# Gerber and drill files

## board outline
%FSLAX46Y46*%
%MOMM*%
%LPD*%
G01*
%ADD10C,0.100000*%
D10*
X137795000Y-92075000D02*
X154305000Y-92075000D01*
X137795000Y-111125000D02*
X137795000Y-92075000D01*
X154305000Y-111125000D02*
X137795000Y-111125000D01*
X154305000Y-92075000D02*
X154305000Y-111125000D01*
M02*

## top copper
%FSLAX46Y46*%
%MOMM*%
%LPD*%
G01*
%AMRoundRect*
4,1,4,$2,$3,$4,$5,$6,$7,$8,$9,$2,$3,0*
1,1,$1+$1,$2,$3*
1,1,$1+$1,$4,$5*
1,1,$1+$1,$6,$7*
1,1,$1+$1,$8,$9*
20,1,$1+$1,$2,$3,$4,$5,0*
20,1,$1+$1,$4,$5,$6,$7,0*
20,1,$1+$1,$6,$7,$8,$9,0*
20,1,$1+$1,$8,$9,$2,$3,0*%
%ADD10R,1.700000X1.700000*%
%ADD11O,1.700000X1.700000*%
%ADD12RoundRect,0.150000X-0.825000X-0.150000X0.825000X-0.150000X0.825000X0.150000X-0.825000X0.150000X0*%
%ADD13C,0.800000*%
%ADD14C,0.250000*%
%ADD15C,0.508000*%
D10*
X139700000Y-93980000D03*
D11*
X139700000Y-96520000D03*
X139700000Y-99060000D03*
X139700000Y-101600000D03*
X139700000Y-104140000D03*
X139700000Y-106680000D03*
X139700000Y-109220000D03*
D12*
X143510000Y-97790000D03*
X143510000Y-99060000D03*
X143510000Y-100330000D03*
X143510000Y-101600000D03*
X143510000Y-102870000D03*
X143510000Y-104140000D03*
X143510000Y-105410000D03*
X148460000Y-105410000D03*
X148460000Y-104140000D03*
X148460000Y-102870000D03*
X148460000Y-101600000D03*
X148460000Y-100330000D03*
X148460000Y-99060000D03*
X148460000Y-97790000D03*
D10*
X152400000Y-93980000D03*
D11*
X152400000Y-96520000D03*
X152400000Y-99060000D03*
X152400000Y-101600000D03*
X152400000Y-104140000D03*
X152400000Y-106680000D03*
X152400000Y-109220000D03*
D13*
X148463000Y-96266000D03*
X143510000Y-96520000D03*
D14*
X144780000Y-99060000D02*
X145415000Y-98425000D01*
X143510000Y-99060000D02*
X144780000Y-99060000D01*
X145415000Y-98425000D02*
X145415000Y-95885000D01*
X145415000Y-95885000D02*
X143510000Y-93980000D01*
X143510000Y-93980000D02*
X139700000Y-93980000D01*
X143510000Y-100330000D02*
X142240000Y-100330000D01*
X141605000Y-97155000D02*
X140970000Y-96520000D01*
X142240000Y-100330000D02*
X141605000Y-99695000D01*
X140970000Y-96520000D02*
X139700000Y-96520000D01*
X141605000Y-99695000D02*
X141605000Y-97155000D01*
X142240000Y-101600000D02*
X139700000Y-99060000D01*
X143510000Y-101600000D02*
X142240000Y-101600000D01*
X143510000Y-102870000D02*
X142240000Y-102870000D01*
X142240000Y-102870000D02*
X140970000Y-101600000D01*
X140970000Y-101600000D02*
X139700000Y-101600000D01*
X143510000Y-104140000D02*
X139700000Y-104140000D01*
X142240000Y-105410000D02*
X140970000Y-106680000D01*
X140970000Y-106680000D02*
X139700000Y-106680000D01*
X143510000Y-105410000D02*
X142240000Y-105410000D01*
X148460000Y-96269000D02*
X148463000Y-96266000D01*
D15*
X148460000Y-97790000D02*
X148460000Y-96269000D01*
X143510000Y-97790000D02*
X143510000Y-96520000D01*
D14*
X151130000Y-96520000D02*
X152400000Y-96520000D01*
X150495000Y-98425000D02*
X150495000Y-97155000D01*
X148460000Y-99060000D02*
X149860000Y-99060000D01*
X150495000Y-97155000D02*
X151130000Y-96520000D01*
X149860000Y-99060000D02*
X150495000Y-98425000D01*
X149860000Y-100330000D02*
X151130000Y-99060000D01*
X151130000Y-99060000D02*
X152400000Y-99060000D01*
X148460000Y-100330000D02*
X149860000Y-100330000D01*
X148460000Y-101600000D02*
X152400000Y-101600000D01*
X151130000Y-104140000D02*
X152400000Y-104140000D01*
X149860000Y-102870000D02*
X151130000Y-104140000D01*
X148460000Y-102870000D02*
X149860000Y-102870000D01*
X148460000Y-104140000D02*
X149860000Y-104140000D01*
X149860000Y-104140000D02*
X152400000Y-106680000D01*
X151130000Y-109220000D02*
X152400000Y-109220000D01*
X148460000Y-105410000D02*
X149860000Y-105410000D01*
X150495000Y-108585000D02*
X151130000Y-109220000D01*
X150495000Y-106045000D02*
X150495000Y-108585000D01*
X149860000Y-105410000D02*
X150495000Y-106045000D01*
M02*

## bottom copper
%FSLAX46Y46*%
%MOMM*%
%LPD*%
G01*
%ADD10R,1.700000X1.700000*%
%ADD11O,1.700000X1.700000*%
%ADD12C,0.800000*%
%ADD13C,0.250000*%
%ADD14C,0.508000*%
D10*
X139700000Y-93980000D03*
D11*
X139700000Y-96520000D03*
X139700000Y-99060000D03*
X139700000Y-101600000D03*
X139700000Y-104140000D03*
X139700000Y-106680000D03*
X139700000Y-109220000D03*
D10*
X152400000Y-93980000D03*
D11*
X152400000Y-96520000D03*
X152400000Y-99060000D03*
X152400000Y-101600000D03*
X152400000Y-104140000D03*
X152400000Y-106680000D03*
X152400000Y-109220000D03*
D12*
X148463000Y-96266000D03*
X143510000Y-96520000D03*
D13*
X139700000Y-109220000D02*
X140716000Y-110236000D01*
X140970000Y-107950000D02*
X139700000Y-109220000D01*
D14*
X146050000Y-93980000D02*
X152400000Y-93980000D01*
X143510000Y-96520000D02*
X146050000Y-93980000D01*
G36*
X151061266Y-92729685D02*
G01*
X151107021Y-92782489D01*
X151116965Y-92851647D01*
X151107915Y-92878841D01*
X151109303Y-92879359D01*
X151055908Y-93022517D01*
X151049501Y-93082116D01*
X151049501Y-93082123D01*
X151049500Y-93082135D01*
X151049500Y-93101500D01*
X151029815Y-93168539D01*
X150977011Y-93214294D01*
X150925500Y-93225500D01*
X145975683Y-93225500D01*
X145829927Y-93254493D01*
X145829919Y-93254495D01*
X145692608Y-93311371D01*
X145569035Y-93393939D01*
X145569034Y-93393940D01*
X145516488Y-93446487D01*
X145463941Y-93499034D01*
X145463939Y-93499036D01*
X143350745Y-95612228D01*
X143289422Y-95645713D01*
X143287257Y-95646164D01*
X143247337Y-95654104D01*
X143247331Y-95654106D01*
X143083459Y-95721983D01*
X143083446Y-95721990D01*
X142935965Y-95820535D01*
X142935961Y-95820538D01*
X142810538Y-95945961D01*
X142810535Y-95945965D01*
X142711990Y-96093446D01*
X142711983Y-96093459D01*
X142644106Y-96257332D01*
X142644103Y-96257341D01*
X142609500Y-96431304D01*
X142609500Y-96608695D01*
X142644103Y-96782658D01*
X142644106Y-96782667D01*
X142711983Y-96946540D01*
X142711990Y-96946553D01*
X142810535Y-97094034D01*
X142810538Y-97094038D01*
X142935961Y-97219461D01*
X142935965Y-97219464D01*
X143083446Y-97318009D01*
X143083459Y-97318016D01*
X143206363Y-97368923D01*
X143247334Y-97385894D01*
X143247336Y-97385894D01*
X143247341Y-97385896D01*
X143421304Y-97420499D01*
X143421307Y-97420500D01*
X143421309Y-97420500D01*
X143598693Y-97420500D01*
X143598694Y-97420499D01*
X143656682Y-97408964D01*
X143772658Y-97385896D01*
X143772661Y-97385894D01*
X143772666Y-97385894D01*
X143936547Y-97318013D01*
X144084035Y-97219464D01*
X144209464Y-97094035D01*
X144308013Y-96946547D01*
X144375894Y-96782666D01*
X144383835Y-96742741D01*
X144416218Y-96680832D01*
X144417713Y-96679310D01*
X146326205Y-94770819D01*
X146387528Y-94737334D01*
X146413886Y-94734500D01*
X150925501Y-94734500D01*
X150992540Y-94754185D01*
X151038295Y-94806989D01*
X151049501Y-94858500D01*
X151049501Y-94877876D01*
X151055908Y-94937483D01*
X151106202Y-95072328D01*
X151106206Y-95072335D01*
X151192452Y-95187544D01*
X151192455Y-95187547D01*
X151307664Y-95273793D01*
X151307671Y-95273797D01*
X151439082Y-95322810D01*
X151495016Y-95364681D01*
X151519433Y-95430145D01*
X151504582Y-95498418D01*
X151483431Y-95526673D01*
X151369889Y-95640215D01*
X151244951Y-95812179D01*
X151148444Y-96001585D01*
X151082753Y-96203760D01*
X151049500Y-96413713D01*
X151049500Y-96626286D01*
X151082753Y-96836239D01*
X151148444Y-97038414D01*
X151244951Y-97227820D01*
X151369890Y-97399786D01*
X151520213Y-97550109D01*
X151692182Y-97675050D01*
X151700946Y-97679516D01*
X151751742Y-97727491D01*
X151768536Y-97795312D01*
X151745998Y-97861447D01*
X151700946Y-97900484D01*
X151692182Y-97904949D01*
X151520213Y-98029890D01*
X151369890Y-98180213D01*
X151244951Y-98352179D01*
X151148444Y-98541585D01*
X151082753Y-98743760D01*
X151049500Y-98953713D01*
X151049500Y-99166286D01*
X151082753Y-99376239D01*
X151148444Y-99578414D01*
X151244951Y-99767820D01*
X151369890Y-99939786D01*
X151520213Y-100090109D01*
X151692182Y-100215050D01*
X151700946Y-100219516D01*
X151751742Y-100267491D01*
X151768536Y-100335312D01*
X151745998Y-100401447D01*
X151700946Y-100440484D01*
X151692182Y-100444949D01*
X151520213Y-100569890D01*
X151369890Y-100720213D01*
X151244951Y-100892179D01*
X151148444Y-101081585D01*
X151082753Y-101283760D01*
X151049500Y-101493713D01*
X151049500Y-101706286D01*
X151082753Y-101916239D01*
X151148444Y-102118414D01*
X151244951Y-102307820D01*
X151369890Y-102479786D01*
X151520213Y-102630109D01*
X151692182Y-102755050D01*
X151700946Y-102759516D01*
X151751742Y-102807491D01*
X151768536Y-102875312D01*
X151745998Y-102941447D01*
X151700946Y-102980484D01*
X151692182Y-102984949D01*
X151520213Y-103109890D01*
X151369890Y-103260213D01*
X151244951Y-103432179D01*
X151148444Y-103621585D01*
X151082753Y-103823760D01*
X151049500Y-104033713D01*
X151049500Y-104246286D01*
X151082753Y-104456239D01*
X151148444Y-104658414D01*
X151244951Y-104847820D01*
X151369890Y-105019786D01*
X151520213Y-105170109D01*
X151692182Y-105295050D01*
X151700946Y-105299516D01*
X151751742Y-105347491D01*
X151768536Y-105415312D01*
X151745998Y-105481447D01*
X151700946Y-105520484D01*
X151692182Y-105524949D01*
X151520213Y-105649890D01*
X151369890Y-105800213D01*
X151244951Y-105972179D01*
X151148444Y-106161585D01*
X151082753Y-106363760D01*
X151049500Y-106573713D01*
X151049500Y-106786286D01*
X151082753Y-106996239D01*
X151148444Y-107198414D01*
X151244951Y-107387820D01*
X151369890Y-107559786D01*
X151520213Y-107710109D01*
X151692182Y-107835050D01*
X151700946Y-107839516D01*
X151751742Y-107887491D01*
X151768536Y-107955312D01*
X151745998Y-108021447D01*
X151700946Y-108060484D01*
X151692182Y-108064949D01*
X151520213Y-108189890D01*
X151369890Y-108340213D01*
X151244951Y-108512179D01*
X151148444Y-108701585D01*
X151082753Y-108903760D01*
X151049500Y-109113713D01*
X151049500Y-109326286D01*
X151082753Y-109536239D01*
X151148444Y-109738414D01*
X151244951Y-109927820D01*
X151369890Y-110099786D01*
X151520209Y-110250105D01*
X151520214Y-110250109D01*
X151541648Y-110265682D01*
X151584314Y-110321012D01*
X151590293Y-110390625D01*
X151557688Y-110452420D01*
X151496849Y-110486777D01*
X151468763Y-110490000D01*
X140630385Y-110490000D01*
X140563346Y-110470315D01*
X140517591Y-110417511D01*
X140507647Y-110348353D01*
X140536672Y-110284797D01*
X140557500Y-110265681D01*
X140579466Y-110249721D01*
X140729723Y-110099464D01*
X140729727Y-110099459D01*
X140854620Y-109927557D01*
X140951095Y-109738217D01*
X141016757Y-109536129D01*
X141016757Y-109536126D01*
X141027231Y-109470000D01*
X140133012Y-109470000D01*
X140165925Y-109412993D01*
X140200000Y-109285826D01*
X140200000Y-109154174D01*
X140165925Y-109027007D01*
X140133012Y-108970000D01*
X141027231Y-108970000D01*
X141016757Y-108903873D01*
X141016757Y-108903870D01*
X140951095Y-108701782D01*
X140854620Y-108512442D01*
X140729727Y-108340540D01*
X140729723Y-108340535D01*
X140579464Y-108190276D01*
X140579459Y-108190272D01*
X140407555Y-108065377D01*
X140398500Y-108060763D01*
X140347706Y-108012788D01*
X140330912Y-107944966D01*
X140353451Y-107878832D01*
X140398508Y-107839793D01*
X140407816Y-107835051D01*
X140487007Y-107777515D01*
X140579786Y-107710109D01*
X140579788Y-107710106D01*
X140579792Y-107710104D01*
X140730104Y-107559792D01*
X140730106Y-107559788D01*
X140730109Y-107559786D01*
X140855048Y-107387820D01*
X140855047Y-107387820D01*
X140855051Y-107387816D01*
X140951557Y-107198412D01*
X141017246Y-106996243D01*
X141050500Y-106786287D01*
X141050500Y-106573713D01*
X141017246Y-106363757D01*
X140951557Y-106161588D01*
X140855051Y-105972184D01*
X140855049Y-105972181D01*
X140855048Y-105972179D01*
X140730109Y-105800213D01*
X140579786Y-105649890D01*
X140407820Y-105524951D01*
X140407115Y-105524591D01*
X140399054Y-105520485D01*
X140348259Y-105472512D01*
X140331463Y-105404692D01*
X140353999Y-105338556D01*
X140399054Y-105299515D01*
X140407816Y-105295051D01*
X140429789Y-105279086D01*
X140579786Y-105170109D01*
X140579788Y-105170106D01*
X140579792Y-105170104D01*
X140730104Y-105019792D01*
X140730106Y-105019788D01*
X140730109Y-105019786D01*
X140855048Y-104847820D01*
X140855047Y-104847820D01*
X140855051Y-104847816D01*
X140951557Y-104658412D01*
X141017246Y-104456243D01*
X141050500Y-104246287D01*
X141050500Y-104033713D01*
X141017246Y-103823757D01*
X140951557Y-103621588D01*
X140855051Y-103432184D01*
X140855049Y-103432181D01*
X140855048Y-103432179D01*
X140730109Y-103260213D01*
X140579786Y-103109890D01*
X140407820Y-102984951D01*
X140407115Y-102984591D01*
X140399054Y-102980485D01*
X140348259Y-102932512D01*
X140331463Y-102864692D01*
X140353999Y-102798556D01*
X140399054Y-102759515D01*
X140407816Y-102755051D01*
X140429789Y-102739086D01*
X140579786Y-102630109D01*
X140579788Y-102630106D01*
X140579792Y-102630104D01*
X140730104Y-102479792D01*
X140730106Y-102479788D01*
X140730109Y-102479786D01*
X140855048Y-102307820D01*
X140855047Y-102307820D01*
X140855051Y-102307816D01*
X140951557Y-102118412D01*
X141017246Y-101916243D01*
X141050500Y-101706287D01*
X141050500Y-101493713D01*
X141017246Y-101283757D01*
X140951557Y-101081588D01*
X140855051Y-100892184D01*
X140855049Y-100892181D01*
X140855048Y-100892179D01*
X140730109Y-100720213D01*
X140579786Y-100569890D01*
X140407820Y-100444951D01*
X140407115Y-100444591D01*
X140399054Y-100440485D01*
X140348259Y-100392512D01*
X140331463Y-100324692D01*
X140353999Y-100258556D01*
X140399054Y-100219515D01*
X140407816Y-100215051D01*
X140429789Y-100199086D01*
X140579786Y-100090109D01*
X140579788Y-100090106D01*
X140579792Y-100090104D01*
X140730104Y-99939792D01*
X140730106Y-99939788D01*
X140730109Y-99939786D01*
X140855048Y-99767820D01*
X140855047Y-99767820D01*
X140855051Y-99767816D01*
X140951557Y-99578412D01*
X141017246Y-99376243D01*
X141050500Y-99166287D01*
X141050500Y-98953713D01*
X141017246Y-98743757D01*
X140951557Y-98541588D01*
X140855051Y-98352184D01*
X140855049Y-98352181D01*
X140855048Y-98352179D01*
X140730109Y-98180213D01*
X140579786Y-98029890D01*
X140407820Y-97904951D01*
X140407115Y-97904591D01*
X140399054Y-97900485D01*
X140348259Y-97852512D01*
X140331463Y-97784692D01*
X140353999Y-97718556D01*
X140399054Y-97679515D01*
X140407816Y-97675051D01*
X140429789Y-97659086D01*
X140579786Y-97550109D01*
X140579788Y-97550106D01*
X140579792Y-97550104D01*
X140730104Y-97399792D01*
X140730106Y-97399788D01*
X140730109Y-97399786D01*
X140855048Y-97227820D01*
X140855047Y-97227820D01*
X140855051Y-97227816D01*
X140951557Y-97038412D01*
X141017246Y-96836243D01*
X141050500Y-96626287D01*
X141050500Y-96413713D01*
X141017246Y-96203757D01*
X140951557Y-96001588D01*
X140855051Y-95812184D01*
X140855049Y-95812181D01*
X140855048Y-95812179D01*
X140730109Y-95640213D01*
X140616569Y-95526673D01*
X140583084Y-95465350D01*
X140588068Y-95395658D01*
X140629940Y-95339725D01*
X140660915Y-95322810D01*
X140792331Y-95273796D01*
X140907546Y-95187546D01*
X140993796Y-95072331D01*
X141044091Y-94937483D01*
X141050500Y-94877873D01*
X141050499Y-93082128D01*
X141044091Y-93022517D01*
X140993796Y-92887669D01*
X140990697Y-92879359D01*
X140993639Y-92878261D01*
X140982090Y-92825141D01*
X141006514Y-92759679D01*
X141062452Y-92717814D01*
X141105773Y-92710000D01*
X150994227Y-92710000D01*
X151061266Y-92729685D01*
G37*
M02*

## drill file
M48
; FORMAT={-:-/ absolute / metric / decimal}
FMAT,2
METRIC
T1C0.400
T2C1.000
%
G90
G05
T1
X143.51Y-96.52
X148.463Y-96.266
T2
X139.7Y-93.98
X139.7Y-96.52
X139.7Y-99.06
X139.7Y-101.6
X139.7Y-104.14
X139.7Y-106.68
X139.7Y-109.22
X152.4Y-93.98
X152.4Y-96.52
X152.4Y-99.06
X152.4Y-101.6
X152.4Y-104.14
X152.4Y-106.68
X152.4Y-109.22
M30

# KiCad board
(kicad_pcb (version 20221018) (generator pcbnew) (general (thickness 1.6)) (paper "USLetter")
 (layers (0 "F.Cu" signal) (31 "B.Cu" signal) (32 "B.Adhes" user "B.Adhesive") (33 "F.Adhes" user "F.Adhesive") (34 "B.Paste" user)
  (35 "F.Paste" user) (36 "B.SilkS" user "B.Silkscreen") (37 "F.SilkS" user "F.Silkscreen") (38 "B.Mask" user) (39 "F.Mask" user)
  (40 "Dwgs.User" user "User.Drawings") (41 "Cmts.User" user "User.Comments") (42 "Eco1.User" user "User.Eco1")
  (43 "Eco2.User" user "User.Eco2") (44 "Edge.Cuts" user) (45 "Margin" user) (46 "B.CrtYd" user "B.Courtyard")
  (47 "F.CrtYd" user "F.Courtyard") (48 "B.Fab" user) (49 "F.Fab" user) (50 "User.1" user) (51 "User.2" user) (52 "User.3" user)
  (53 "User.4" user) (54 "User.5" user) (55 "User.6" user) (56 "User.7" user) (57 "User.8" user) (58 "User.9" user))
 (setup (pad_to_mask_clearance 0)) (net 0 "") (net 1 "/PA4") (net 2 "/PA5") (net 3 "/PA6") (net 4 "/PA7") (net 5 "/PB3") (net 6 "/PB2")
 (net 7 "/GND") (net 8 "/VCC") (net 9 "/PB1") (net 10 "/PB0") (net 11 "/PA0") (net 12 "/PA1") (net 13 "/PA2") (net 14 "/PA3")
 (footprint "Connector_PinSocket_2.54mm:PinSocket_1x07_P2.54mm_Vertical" (layer "F.Cu") (at 139.7 93.98)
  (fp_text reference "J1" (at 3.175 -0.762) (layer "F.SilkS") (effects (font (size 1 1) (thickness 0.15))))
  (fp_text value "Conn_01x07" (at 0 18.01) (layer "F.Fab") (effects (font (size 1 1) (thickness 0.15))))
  (pad "1" thru_hole rect (at 0 0) (size 1.7 1.7) (drill 1) (layers "*.Cu" "*.Mask") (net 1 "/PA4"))
  (pad "2" thru_hole oval (at 0 2.54) (size 1.7 1.7) (drill 1) (layers "*.Cu" "*.Mask") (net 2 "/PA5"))
  (pad "3" thru_hole oval (at 0 5.08) (size 1.7 1.7) (drill 1) (layers "*.Cu" "*.Mask") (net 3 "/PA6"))
  (pad "4" thru_hole oval (at 0 7.62) (size 1.7 1.7) (drill 1) (layers "*.Cu" "*.Mask") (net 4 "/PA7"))
  (pad "5" thru_hole oval (at 0 10.16) (size 1.7 1.7) (drill 1) (layers "*.Cu" "*.Mask") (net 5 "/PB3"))
  (pad "6" thru_hole oval (at 0 12.7) (size 1.7 1.7) (drill 1) (layers "*.Cu" "*.Mask") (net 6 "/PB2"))
  (pad "7" thru_hole oval (at 0 15.24) (size 1.7 1.7) (drill 1) (layers "*.Cu" "*.Mask") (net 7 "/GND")))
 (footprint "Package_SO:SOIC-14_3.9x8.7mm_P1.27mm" (layer "F.Cu") (at 145.985 101.6)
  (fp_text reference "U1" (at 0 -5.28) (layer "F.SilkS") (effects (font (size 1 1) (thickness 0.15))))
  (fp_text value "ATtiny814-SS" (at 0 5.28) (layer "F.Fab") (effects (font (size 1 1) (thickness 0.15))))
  (pad "1" smd roundrect (at -2.475 -3.81) (size 1.95 0.6) (layers "F.Cu" "F.Paste" "F.Mask") (roundrect_rratio 0.25) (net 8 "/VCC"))
  (pad "2" smd roundrect (at -2.475 -2.54) (size 1.95 0.6) (layers "F.Cu" "F.Paste" "F.Mask") (roundrect_rratio 0.25) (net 1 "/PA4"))
  (pad "3" smd roundrect (at -2.475 -1.27) (size 1.95 0.6) (layers "F.Cu" "F.Paste" "F.Mask") (roundrect_rratio 0.25) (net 2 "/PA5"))
  (pad "4" smd roundrect (at -2.475 0) (size 1.95 0.6) (layers "F.Cu" "F.Paste" "F.Mask") (roundrect_rratio 0.25) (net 3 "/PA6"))
  (pad "5" smd roundrect (at -2.475 1.27) (size 1.95 0.6) (layers "F.Cu" "F.Paste" "F.Mask") (roundrect_rratio 0.25) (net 4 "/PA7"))
  (pad "6" smd roundrect (at -2.475 2.54) (size 1.95 0.6) (layers "F.Cu" "F.Paste" "F.Mask") (roundrect_rratio 0.25) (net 5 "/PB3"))
  (pad "7" smd roundrect (at -2.475 3.81) (size 1.95 0.6) (layers "F.Cu" "F.Paste" "F.Mask") (roundrect_rratio 0.25) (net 6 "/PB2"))
  (pad "8" smd roundrect (at 2.475 3.81) (size 1.95 0.6) (layers "F.Cu" "F.Paste" "F.Mask") (roundrect_rratio 0.25) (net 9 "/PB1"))
  (pad "9" smd roundrect (at 2.475 2.54) (size 1.95 0.6) (layers "F.Cu" "F.Paste" "F.Mask") (roundrect_rratio 0.25) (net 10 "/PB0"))
  (pad "10" smd roundrect (at 2.475 1.27) (size 1.95 0.6) (layers "F.Cu" "F.Paste" "F.Mask") (roundrect_rratio 0.25) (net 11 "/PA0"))
  (pad "11" smd roundrect (at 2.475 0) (size 1.95 0.6) (layers "F.Cu" "F.Paste" "F.Mask") (roundrect_rratio 0.25) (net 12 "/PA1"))
  (pad "12" smd roundrect (at 2.475 -1.27) (size 1.95 0.6) (layers "F.Cu" "F.Paste" "F.Mask") (roundrect_rratio 0.25) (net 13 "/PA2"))
  (pad "13" smd roundrect (at 2.475 -2.54) (size 1.95 0.6) (layers "F.Cu" "F.Paste" "F.Mask") (roundrect_rratio 0.25) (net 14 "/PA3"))
  (pad "14" smd roundrect (at 2.475 -3.81) (size 1.95 0.6) (layers "F.Cu" "F.Paste" "F.Mask") (roundrect_rratio 0.25) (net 7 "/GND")))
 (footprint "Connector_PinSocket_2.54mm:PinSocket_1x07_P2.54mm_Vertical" (layer "F.Cu") (at 152.4 93.98)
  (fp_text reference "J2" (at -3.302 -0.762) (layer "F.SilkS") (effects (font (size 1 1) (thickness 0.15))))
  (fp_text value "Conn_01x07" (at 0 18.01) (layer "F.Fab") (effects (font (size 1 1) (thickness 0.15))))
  (pad "1" thru_hole rect (at 0 0) (size 1.7 1.7) (drill 1) (layers "*.Cu" "*.Mask") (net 8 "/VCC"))
  (pad "2" thru_hole oval (at 0 2.54) (size 1.7 1.7) (drill 1) (layers "*.Cu" "*.Mask") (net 14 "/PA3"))
  (pad "3" thru_hole oval (at 0 5.08) (size 1.7 1.7) (drill 1) (layers "*.Cu" "*.Mask") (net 13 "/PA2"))
  (pad "4" thru_hole oval (at 0 7.62) (size 1.7 1.7) (drill 1) (layers "*.Cu" "*.Mask") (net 12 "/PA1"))
  (pad "5" thru_hole oval (at 0 10.16) (size 1.7 1.7) (drill 1) (layers "*.Cu" "*.Mask") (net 11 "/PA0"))
  (pad "6" thru_hole oval (at 0 12.7) (size 1.7 1.7) (drill 1) (layers "*.Cu" "*.Mask") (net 10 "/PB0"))
  (pad "7" thru_hole oval (at 0 15.24) (size 1.7 1.7) (drill 1) (layers "*.Cu" "*.Mask") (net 9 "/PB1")))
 (gr_line (start 137.795 92.075) (end 154.305 92.075) (stroke (width 0.1) (type default)) (layer "Edge.Cuts"))
 (gr_line (start 137.795 111.125) (end 137.795 92.075) (stroke (width 0.1) (type default)) (layer "Edge.Cuts"))
 (gr_line (start 154.305 111.125) (end 137.795 111.125) (stroke (width 0.1) (type default)) (layer "Edge.Cuts"))
 (gr_line (start 154.305 92.075) (end 154.305 111.125) (stroke (width 0.1) (type default)) (layer "Edge.Cuts"))
 (segment (start 144.78 99.06) (end 145.415 98.425) (width 0.25) (layer "F.Cu") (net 1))
 (segment (start 143.51 99.06) (end 144.78 99.06) (width 0.25) (layer "F.Cu") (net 1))
 (segment (start 145.415 98.425) (end 145.415 95.885) (width 0.25) (layer "F.Cu") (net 1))
 (segment (start 145.415 95.885) (end 143.51 93.98) (width 0.25) (layer "F.Cu") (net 1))
 (segment (start 143.51 93.98) (end 139.7 93.98) (width 0.25) (layer "F.Cu") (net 1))
 (segment (start 143.51 100.33) (end 142.24 100.33) (width 0.25) (layer "F.Cu") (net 2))
 (segment (start 141.605 97.155) (end 140.97 96.52) (width 0.25) (layer "F.Cu") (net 2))
 (segment (start 142.24 100.33) (end 141.605 99.695) (width 0.25) (layer "F.Cu") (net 2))
 (segment (start 140.97 96.52) (end 139.7 96.52) (width 0.25) (layer "F.Cu") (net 2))
 (segment (start 141.605 99.695) (end 141.605 97.155) (width 0.25) (layer "F.Cu") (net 2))
 (segment (start 142.24 101.6) (end 139.7 99.06) (width 0.25) (layer "F.Cu") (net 3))
 (segment (start 143.51 101.6) (end 142.24 101.6) (width 0.25) (layer "F.Cu") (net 3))
 (segment (start 143.51 102.87) (end 142.24 102.87) (width 0.25) (layer "F.Cu") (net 4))
 (segment (start 142.24 102.87) (end 140.97 101.6) (width 0.25) (layer "F.Cu") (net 4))
 (segment (start 140.97 101.6) (end 139.7 101.6) (width 0.25) (layer "F.Cu") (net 4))
 (segment (start 143.51 104.14) (end 139.7 104.14) (width 0.25) (layer "F.Cu") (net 5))
 (segment (start 142.24 105.41) (end 140.97 106.68) (width 0.25) (layer "F.Cu") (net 6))
 (segment (start 140.97 106.68) (end 139.7 106.68) (width 0.25) (layer "F.Cu") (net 6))
 (segment (start 143.51 105.41) (end 142.24 105.41) (width 0.25) (layer "F.Cu") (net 6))
 (segment (start 148.46 96.269) (end 148.463 96.266) (width 0.25) (layer "F.Cu") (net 7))
 (segment (start 148.46 97.79) (end 148.46 96.269) (width 0.508) (layer "F.Cu") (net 7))
 (via (at 148.463 96.266) (size 0.8) (drill 0.4) (layers "F.Cu" "B.Cu") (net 7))
 (segment (start 139.7 109.22) (end 140.716 110.236) (width 0.25) (layer "B.Cu") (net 7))
 (segment (start 140.97 107.95) (end 139.7 109.22) (width 0.25) (layer "B.Cu") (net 7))
 (segment (start 143.51 97.79) (end 143.51 96.52) (width 0.508) (layer "F.Cu") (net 8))
 (via (at 143.51 96.52) (size 0.8) (drill 0.4) (layers "F.Cu" "B.Cu") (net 8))
 (segment (start 146.05 93.98) (end 152.4 93.98) (width 0.508) (layer "B.Cu") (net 8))
 (segment (start 143.51 96.52) (end 146.05 93.98) (width 0.508) (layer "B.Cu") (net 8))
 (segment (start 151.13 96.52) (end 152.4 96.52) (width 0.25) (layer "F.Cu") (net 14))
 (segment (start 150.495 98.425) (end 150.495 97.155) (width 0.25) (layer "F.Cu") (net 14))
 (segment (start 148.46 99.06) (end 149.86 99.06) (width 0.25) (layer "F.Cu") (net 14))
 (segment (start 150.495 97.155) (end 151.13 96.52) (width 0.25) (layer "F.Cu") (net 14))
 (segment (start 149.86 99.06) (end 150.495 98.425) (width 0.25) (layer "F.Cu") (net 14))
 (segment (start 149.86 100.33) (end 151.13 99.06) (width 0.25) (layer "F.Cu") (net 13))
 (segment (start 151.13 99.06) (end 152.4 99.06) (width 0.25) (layer "F.Cu") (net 13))
 (segment (start 148.46 100.33) (end 149.86 100.33) (width 0.25) (layer "F.Cu") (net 13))
 (segment (start 148.46 101.6) (end 152.4 101.6) (width 0.25) (layer "F.Cu") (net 12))
 (segment (start 151.13 104.14) (end 152.4 104.14) (width 0.25) (layer "F.Cu") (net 11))
 (segment (start 149.86 102.87) (end 151.13 104.14) (width 0.25) (layer "F.Cu") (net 11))
 (segment (start 148.46 102.87) (end 149.86 102.87) (width 0.25) (layer "F.Cu") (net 11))
 (segment (start 148.46 104.14) (end 149.86 104.14) (width 0.25) (layer "F.Cu") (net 10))
 (segment (start 149.86 104.14) (end 152.4 106.68) (width 0.25) (layer "F.Cu") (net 10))
 (segment (start 151.13 109.22) (end 152.4 109.22) (width 0.25) (layer "F.Cu") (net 9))
 (segment (start 148.46 105.41) (end 149.86 105.41) (width 0.25) (layer "F.Cu") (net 9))
 (segment (start 150.495 108.585) (end 151.13 109.22) (width 0.25) (layer "F.Cu") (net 9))
 (segment (start 150.495 106.045) (end 150.495 108.585) (width 0.25) (layer "F.Cu") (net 9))
 (segment (start 149.86 105.41) (end 150.495 106.045) (width 0.25) (layer "F.Cu") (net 9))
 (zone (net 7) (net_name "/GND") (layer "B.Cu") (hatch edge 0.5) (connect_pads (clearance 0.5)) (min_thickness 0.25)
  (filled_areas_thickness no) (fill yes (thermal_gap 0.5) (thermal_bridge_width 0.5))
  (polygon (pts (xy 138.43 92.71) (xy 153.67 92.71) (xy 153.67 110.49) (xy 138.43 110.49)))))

